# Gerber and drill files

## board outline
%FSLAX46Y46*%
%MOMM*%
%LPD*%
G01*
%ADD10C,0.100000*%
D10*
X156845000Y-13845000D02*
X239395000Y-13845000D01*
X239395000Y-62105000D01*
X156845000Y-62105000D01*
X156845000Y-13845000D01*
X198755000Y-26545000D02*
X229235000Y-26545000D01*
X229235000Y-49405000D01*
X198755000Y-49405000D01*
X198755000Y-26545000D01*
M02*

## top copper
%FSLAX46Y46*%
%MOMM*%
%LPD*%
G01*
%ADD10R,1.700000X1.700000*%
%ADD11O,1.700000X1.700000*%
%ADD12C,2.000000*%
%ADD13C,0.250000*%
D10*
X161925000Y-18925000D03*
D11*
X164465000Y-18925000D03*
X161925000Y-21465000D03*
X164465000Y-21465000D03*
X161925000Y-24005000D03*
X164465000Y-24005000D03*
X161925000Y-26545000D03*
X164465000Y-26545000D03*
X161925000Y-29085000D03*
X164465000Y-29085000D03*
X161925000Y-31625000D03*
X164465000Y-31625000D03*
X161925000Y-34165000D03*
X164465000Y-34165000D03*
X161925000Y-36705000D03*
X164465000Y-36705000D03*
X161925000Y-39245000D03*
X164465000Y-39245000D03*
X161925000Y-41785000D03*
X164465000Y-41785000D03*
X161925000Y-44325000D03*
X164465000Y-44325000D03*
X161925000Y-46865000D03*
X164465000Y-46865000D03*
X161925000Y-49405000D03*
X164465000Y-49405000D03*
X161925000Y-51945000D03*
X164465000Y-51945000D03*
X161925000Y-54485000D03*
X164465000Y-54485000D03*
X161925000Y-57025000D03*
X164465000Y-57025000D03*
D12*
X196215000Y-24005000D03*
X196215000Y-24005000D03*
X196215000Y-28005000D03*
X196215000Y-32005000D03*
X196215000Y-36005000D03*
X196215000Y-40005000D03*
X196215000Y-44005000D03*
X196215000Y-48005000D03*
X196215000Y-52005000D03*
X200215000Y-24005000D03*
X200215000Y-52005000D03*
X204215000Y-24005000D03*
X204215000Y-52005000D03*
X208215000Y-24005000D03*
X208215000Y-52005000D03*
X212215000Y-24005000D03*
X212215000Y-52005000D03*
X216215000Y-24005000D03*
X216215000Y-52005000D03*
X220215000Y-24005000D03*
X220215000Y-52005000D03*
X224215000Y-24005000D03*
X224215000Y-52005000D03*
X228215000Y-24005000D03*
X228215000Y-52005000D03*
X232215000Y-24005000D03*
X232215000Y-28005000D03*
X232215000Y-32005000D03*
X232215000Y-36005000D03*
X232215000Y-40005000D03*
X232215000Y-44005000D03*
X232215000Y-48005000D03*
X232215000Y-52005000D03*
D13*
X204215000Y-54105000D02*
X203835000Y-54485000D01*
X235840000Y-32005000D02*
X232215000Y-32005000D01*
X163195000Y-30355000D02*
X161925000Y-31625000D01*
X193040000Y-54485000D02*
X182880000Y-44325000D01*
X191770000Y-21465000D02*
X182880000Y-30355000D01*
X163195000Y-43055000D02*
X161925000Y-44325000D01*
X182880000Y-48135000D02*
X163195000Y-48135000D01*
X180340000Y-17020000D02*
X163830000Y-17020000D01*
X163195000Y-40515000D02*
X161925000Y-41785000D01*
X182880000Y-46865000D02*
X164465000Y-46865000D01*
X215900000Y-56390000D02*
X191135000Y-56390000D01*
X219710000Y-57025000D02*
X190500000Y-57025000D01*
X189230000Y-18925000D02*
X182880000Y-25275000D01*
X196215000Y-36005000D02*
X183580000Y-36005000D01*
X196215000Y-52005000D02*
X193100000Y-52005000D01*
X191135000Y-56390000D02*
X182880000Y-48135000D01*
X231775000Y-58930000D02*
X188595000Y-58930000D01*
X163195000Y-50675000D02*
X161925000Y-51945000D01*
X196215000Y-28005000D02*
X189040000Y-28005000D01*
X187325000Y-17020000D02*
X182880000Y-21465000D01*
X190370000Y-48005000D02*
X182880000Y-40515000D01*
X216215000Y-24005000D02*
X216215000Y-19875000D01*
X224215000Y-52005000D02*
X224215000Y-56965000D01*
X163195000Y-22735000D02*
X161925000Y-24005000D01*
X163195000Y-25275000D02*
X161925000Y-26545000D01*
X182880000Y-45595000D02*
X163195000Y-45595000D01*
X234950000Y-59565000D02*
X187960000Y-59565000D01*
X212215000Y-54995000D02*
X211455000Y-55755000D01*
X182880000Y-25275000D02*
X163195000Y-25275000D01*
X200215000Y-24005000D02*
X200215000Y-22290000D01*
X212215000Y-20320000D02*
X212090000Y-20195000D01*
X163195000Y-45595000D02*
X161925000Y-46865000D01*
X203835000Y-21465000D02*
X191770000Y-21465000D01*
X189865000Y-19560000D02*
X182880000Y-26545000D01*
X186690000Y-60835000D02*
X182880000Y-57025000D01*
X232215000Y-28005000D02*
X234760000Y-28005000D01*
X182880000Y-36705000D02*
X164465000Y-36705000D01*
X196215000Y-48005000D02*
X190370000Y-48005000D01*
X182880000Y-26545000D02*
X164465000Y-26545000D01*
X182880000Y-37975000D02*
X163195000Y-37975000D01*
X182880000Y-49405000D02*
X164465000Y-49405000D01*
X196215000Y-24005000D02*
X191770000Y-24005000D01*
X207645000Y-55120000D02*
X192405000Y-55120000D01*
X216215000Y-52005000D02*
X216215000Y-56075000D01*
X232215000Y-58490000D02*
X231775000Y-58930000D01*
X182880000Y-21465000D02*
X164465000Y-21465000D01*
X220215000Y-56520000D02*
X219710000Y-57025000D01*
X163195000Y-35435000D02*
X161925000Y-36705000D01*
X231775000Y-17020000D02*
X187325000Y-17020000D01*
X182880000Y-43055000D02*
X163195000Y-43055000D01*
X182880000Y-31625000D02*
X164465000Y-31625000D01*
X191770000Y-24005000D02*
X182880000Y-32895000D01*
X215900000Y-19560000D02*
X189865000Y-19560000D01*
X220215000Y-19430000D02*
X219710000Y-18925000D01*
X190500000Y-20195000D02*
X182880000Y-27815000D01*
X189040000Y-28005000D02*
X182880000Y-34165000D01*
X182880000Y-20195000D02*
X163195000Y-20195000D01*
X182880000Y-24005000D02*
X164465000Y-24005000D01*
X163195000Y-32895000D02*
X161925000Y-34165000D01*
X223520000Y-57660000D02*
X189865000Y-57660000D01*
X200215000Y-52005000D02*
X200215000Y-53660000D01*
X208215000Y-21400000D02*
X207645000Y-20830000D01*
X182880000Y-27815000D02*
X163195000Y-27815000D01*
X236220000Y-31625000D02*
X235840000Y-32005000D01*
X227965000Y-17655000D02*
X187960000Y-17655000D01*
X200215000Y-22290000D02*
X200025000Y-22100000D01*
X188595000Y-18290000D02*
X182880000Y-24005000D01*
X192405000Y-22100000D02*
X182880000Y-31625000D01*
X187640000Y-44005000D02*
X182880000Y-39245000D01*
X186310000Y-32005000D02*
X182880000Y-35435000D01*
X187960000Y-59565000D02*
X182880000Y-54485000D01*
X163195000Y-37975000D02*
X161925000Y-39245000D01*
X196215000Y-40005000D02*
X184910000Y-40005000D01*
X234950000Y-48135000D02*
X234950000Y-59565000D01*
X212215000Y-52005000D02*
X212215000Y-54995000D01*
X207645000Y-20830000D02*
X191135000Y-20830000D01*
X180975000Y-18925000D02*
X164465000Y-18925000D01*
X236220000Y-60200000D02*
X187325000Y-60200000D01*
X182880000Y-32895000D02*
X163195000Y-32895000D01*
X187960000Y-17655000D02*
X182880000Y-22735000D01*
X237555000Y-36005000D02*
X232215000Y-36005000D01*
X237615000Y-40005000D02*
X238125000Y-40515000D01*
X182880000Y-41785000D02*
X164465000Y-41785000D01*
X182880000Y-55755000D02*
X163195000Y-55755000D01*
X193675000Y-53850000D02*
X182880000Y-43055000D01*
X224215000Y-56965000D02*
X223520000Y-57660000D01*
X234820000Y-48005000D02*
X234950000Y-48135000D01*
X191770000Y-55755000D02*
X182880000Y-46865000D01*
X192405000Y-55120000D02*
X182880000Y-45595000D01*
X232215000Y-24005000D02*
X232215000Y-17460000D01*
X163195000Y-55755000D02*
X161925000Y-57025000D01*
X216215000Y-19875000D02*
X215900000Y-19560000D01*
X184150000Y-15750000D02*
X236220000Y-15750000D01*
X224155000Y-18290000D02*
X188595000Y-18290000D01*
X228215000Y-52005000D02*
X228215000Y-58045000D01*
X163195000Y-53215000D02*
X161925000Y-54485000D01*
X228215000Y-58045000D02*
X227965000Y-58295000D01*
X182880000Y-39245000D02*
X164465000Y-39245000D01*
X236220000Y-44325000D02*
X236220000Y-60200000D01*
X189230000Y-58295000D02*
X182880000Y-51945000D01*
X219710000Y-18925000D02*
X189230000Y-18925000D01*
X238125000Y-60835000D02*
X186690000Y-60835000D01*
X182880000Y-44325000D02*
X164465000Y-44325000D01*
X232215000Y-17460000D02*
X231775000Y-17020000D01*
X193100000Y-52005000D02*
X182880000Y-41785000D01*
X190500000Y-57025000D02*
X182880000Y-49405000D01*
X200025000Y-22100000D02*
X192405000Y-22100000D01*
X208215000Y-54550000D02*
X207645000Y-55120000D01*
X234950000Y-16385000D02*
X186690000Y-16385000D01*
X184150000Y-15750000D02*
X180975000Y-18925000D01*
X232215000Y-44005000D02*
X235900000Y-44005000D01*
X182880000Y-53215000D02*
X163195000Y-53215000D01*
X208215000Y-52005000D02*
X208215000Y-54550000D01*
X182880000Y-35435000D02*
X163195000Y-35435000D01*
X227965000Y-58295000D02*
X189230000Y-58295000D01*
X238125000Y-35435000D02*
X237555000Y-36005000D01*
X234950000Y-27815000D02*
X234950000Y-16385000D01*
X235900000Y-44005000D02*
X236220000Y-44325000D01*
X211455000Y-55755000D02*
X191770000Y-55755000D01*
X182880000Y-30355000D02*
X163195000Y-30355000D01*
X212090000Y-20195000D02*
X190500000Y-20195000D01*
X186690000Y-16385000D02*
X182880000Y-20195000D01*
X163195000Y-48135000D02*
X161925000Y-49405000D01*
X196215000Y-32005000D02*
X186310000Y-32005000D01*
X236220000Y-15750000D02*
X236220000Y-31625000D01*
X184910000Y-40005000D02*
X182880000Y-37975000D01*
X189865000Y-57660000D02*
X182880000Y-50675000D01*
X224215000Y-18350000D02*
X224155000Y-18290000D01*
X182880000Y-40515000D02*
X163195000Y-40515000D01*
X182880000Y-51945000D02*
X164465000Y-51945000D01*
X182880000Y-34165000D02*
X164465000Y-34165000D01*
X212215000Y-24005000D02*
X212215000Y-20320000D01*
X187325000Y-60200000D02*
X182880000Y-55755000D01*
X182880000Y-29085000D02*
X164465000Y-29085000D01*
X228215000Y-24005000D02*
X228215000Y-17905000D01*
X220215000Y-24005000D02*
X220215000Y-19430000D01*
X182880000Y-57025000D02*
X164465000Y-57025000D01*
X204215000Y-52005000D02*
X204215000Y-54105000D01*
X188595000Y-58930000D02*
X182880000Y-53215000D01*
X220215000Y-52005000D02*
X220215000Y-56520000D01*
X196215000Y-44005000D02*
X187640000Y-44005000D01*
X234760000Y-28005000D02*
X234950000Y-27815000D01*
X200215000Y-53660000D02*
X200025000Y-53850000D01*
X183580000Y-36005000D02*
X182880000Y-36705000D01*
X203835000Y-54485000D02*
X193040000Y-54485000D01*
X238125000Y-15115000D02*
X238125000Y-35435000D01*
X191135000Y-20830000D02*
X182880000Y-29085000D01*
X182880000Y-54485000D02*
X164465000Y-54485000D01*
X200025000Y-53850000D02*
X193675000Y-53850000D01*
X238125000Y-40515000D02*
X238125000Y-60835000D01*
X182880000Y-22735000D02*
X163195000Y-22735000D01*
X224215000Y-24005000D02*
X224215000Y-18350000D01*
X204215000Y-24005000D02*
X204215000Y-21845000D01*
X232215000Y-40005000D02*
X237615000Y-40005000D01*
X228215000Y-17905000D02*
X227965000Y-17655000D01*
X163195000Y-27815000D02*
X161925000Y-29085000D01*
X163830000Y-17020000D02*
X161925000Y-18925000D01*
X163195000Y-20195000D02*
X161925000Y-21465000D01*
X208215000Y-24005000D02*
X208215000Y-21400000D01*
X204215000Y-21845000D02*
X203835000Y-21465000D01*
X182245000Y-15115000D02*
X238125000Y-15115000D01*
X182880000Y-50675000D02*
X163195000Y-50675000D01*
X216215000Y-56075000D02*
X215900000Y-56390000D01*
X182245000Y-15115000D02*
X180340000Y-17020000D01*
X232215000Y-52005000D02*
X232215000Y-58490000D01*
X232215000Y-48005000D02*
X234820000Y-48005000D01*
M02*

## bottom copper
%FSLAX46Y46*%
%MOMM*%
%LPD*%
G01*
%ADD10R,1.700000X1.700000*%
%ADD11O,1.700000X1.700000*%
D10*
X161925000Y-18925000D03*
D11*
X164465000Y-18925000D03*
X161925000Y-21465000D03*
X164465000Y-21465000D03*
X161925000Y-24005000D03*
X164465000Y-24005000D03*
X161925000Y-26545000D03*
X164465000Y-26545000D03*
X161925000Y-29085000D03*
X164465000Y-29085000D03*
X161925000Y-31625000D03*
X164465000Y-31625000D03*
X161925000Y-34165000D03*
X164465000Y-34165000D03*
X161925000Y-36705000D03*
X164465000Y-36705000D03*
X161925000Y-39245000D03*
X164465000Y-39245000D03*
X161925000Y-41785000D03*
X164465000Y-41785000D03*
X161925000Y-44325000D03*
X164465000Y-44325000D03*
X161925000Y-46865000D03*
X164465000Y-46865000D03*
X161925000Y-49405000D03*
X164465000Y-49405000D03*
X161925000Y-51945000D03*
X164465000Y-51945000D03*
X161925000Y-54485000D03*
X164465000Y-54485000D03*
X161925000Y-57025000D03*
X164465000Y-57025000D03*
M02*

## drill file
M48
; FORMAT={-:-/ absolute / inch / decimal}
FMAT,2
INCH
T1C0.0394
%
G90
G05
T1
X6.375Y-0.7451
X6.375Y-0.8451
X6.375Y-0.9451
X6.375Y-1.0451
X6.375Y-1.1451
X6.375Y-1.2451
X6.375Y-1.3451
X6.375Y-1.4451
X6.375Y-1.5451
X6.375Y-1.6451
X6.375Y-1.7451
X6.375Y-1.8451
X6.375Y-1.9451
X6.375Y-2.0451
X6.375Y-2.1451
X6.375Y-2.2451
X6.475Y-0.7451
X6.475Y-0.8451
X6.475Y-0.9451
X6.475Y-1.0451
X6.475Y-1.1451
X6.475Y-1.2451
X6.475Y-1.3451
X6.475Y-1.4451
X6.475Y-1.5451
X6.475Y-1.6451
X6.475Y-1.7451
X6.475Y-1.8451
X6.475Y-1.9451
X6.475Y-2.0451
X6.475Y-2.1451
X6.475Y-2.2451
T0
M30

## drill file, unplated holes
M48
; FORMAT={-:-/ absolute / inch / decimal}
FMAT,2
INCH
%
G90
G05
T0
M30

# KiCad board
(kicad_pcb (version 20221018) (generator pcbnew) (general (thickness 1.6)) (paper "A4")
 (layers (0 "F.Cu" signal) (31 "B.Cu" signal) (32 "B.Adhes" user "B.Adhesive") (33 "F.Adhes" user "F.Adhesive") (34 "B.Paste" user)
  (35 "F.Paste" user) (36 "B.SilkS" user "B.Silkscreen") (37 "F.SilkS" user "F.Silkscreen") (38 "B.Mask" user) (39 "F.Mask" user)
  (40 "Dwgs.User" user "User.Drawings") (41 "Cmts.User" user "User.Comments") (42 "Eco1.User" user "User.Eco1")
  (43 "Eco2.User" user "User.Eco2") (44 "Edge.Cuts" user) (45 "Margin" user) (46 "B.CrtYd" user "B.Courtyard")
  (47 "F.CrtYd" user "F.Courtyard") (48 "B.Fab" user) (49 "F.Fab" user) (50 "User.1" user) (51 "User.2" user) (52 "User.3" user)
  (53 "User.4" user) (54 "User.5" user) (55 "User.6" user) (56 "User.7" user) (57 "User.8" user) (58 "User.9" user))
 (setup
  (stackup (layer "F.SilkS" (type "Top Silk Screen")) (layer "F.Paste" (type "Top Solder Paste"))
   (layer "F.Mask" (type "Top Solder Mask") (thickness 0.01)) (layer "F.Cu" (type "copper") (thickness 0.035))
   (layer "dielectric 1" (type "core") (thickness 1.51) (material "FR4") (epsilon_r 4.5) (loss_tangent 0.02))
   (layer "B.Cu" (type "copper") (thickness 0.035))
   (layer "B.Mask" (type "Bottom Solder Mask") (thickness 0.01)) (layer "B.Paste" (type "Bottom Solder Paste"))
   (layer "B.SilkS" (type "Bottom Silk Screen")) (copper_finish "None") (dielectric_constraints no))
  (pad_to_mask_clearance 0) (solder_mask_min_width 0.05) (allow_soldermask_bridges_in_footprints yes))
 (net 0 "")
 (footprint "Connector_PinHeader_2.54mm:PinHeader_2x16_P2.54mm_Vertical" (layer "F.Cu") (at 161.925 18.925)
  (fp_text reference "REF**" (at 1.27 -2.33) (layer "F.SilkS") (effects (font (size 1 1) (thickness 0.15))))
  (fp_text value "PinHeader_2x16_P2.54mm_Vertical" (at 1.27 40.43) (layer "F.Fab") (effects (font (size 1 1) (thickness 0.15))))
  (pad "1" thru_hole rect (at 0 0) (size 1.7 1.7) (drill 1) (layers "*.Cu" "*.Mask"))
  (pad "2" thru_hole oval (at 2.54 0) (size 1.7 1.7) (drill 1) (layers "*.Cu" "*.Mask"))
  (pad "3" thru_hole oval (at 0 2.54) (size 1.7 1.7) (drill 1) (layers "*.Cu" "*.Mask"))
  (pad "4" thru_hole oval (at 2.54 2.54) (size 1.7 1.7) (drill 1) (layers "*.Cu" "*.Mask"))
  (pad "5" thru_hole oval (at 0 5.08) (size 1.7 1.7) (drill 1) (layers "*.Cu" "*.Mask"))
  (pad "6" thru_hole oval (at 2.54 5.08) (size 1.7 1.7) (drill 1) (layers "*.Cu" "*.Mask"))
  (pad "7" thru_hole oval (at 0 7.62) (size 1.7 1.7) (drill 1) (layers "*.Cu" "*.Mask"))
  (pad "8" thru_hole oval (at 2.54 7.62) (size 1.7 1.7) (drill 1) (layers "*.Cu" "*.Mask"))
  (pad "9" thru_hole oval (at 0 10.16) (size 1.7 1.7) (drill 1) (layers "*.Cu" "*.Mask"))
  (pad "10" thru_hole oval (at 2.54 10.16) (size 1.7 1.7) (drill 1) (layers "*.Cu" "*.Mask"))
  (pad "11" thru_hole oval (at 0 12.7) (size 1.7 1.7) (drill 1) (layers "*.Cu" "*.Mask") (clearance 0.2))
  (pad "12" thru_hole oval (at 2.54 12.7) (size 1.7 1.7) (drill 1) (layers "*.Cu" "*.Mask"))
  (pad "13" thru_hole oval (at 0 15.24) (size 1.7 1.7) (drill 1) (layers "*.Cu" "*.Mask"))
  (pad "14" thru_hole oval (at 2.54 15.24) (size 1.7 1.7) (drill 1) (layers "*.Cu" "*.Mask"))
  (pad "15" thru_hole oval (at 0 17.78) (size 1.7 1.7) (drill 1) (layers "*.Cu" "*.Mask"))
  (pad "16" thru_hole oval (at 2.54 17.78) (size 1.7 1.7) (drill 1) (layers "*.Cu" "*.Mask"))
  (pad "17" thru_hole oval (at 0 20.32) (size 1.7 1.7) (drill 1) (layers "*.Cu" "*.Mask"))
  (pad "18" thru_hole oval (at 2.54 20.32) (size 1.7 1.7) (drill 1) (layers "*.Cu" "*.Mask"))
  (pad "19" thru_hole oval (at 0 22.86) (size 1.7 1.7) (drill 1) (layers "*.Cu" "*.Mask"))
  (pad "20" thru_hole oval (at 2.54 22.86) (size 1.7 1.7) (drill 1) (layers "*.Cu" "*.Mask"))
  (pad "21" thru_hole oval (at 0 25.4) (size 1.7 1.7) (drill 1) (layers "*.Cu" "*.Mask"))
  (pad "22" thru_hole oval (at 2.54 25.4) (size 1.7 1.7) (drill 1) (layers "*.Cu" "*.Mask"))
  (pad "23" thru_hole oval (at 0 27.94) (size 1.7 1.7) (drill 1) (layers "*.Cu" "*.Mask"))
  (pad "24" thru_hole oval (at 2.54 27.94) (size 1.7 1.7) (drill 1) (layers "*.Cu" "*.Mask"))
  (pad "25" thru_hole oval (at 0 30.48) (size 1.7 1.7) (drill 1) (layers "*.Cu" "*.Mask"))
  (pad "26" thru_hole oval (at 2.54 30.48) (size 1.7 1.7) (drill 1) (layers "*.Cu" "*.Mask"))
  (pad "27" thru_hole oval (at 0 33.02) (size 1.7 1.7) (drill 1) (layers "*.Cu" "*.Mask"))
  (pad "28" thru_hole oval (at 2.54 33.02) (size 1.7 1.7) (drill 1) (layers "*.Cu" "*.Mask"))
  (pad "29" thru_hole oval (at 0 35.56) (size 1.7 1.7) (drill 1) (layers "*.Cu" "*.Mask"))
  (pad "30" thru_hole oval (at 2.54 35.56) (size 1.7 1.7) (drill 1) (layers "*.Cu" "*.Mask"))
  (pad "31" thru_hole oval (at 0 38.1) (size 1.7 1.7) (drill 1) (layers "*.Cu" "*.Mask"))
  (pad "32" thru_hole oval (at 2.54 38.1) (size 1.7 1.7) (drill 1) (layers "*.Cu" "*.Mask")))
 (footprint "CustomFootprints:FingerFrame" (layer "F.Cu") (at 196.215 24.005)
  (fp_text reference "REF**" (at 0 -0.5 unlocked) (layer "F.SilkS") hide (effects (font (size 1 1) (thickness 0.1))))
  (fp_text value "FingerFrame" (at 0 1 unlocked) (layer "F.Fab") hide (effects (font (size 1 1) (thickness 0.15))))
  (pad "1" smd circle (at 0 0) (size 2 2) (layers "F.Cu" "F.Paste" "F.Mask"))
  (pad "1" smd circle (at 0 0) (size 2 2) (layers "F.Cu" "F.Paste" "F.Mask"))
  (pad "1" smd circle (at 0 4) (size 2 2) (layers "F.Cu" "F.Paste" "F.Mask"))
  (pad "1" smd circle (at 0 8) (size 2 2) (layers "F.Cu" "F.Paste" "F.Mask"))
  (pad "1" smd circle (at 0 12) (size 2 2) (layers "F.Cu" "F.Paste" "F.Mask"))
  (pad "1" smd circle (at 0 16) (size 2 2) (layers "F.Cu" "F.Paste" "F.Mask"))
  (pad "1" smd circle (at 0 20) (size 2 2) (layers "F.Cu" "F.Paste" "F.Mask"))
  (pad "1" smd circle (at 0 24) (size 2 2) (layers "F.Cu" "F.Paste" "F.Mask"))
  (pad "1" smd circle (at 0 28) (size 2 2) (layers "F.Cu" "F.Paste" "F.Mask"))
  (pad "1" smd circle (at 4 0) (size 2 2) (layers "F.Cu" "F.Paste" "F.Mask"))
  (pad "1" smd circle (at 4 28) (size 2 2) (layers "F.Cu" "F.Paste" "F.Mask"))
  (pad "1" smd circle (at 8 0) (size 2 2) (layers "F.Cu" "F.Paste" "F.Mask"))
  (pad "1" smd circle (at 8 28) (size 2 2) (layers "F.Cu" "F.Paste" "F.Mask"))
  (pad "1" smd circle (at 12 0) (size 2 2) (layers "F.Cu" "F.Paste" "F.Mask"))
  (pad "1" smd circle (at 12 28) (size 2 2) (layers "F.Cu" "F.Paste" "F.Mask"))
  (pad "1" smd circle (at 16 0) (size 2 2) (layers "F.Cu" "F.Paste" "F.Mask"))
  (pad "1" smd circle (at 16 28) (size 2 2) (layers "F.Cu" "F.Paste" "F.Mask"))
  (pad "1" smd circle (at 20 0) (size 2 2) (layers "F.Cu" "F.Paste" "F.Mask"))
  (pad "1" smd circle (at 20 28) (size 2 2) (layers "F.Cu" "F.Paste" "F.Mask"))
  (pad "1" smd circle (at 24 0) (size 2 2) (layers "F.Cu" "F.Paste" "F.Mask"))
  (pad "1" smd circle (at 24 28) (size 2 2) (layers "F.Cu" "F.Paste" "F.Mask"))
  (pad "1" smd circle (at 28 0) (size 2 2) (layers "F.Cu" "F.Paste" "F.Mask"))
  (pad "1" smd circle (at 28 28) (size 2 2) (layers "F.Cu" "F.Paste" "F.Mask"))
  (pad "1" smd circle (at 32 0) (size 2 2) (layers "F.Cu" "F.Paste" "F.Mask"))
  (pad "1" smd circle (at 32 28) (size 2 2) (layers "F.Cu" "F.Paste" "F.Mask"))
  (pad "1" smd circle (at 36 0) (size 2 2) (layers "F.Cu" "F.Paste" "F.Mask"))
  (pad "1" smd circle (at 36 4) (size 2 2) (layers "F.Cu" "F.Paste" "F.Mask"))
  (pad "1" smd circle (at 36 8) (size 2 2) (layers "F.Cu" "F.Paste" "F.Mask"))
  (pad "1" smd circle (at 36 12) (size 2 2) (layers "F.Cu" "F.Paste" "F.Mask"))
  (pad "1" smd circle (at 36 16) (size 2 2) (layers "F.Cu" "F.Paste" "F.Mask"))
  (pad "1" smd circle (at 36 20) (size 2 2) (layers "F.Cu" "F.Paste" "F.Mask"))
  (pad "1" smd circle (at 36 24) (size 2 2) (layers "F.Cu" "F.Paste" "F.Mask"))
  (pad "1" smd circle (at 36 28) (size 2 2) (layers "F.Cu" "F.Paste" "F.Mask")))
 (gr_rect (start 156.845 13.845) (end 239.395 62.105) (stroke (width 0.1) (type default)) (fill none) (layer "Edge.Cuts"))
 (gr_rect (start 198.755 26.545) (end 229.235 49.405) (stroke (width 0.1) (type default)) (fill none) (layer "Edge.Cuts"))
 (segment (start 204.215 54.105) (end 203.835 54.485) (width 0.25) (layer "F.Cu") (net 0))
 (segment (start 235.84 32.005) (end 232.215 32.005) (width 0.25) (layer "F.Cu") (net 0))
 (segment (start 163.195 30.355) (end 161.925 31.625) (width 0.25) (layer "F.Cu") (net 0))
 (segment (start 193.04 54.485) (end 182.88 44.325) (width 0.25) (layer "F.Cu") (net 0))
 (segment (start 191.77 21.465) (end 182.88 30.355) (width 0.25) (layer "F.Cu") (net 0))
 (segment (start 163.195 43.055) (end 161.925 44.325) (width 0.25) (layer "F.Cu") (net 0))
 (segment (start 182.88 48.135) (end 163.195 48.135) (width 0.25) (layer "F.Cu") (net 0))
 (segment (start 180.34 17.02) (end 163.83 17.02) (width 0.25) (layer "F.Cu") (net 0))
 (segment (start 163.195 40.515) (end 161.925 41.785) (width 0.25) (layer "F.Cu") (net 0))
 (segment (start 182.88 46.865) (end 164.465 46.865) (width 0.25) (layer "F.Cu") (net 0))
 (segment (start 215.9 56.39) (end 191.135 56.39) (width 0.25) (layer "F.Cu") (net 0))
 (segment (start 219.71 57.025) (end 190.5 57.025) (width 0.25) (layer "F.Cu") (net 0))
 (segment (start 189.23 18.925) (end 182.88 25.275) (width 0.25) (layer "F.Cu") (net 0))
 (segment (start 196.215 36.005) (end 183.58 36.005) (width 0.25) (layer "F.Cu") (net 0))
 (segment (start 196.215 52.005) (end 193.1 52.005) (width 0.25) (layer "F.Cu") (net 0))
 (segment (start 191.135 56.39) (end 182.88 48.135) (width 0.25) (layer "F.Cu") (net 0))
 (segment (start 231.775 58.93) (end 188.595 58.93) (width 0.25) (layer "F.Cu") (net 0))
 (segment (start 163.195 50.675) (end 161.925 51.945) (width 0.25) (layer "F.Cu") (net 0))
 (segment (start 196.215 28.005) (end 189.04 28.005) (width 0.25) (layer "F.Cu") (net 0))
 (segment (start 187.325 17.02) (end 182.88 21.465) (width 0.25) (layer "F.Cu") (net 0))
 (segment (start 190.37 48.005) (end 182.88 40.515) (width 0.25) (layer "F.Cu") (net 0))
 (segment (start 216.215 24.005) (end 216.215 19.875) (width 0.25) (layer "F.Cu") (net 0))
 (segment (start 224.215 52.005) (end 224.215 56.965) (width 0.25) (layer "F.Cu") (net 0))
 (segment (start 163.195 22.735) (end 161.925 24.005) (width 0.25) (layer "F.Cu") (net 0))
 (segment (start 163.195 25.275) (end 161.925 26.545) (width 0.25) (layer "F.Cu") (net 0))
 (segment (start 182.88 45.595) (end 163.195 45.595) (width 0.25) (layer "F.Cu") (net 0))
 (segment (start 234.95 59.565) (end 187.96 59.565) (width 0.25) (layer "F.Cu") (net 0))
 (segment (start 212.215 54.995) (end 211.455 55.755) (width 0.25) (layer "F.Cu") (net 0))
 (segment (start 182.88 25.275) (end 163.195 25.275) (width 0.25) (layer "F.Cu") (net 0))
 (segment (start 200.215 24.005) (end 200.215 22.29) (width 0.25) (layer "F.Cu") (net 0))
 (segment (start 212.215 20.32) (end 212.09 20.195) (width 0.25) (layer "F.Cu") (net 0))
 (segment (start 163.195 45.595) (end 161.925 46.865) (width 0.25) (layer "F.Cu") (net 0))
 (segment (start 203.835 21.465) (end 191.77 21.465) (width 0.25) (layer "F.Cu") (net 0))
 (segment (start 189.865 19.56) (end 182.88 26.545) (width 0.25) (layer "F.Cu") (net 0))
 (segment (start 186.69 60.835) (end 182.88 57.025) (width 0.25) (layer "F.Cu") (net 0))
 (segment (start 232.215 28.005) (end 234.76 28.005) (width 0.25) (layer "F.Cu") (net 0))
 (segment (start 182.88 36.705) (end 164.465 36.705) (width 0.25) (layer "F.Cu") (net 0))
 (segment (start 196.215 48.005) (end 190.37 48.005) (width 0.25) (layer "F.Cu") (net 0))
 (segment (start 182.88 26.545) (end 164.465 26.545) (width 0.25) (layer "F.Cu") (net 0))
 (segment (start 182.88 37.975) (end 163.195 37.975) (width 0.25) (layer "F.Cu") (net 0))
 (segment (start 182.88 49.405) (end 164.465 49.405) (width 0.25) (layer "F.Cu") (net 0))
 (segment (start 196.215 24.005) (end 191.77 24.005) (width 0.25) (layer "F.Cu") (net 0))
 (segment (start 207.645 55.12) (end 192.405 55.12) (width 0.25) (layer "F.Cu") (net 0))
 (segment (start 216.215 52.005) (end 216.215 56.075) (width 0.25) (layer "F.Cu") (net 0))
 (segment (start 232.215 58.49) (end 231.775 58.93) (width 0.25) (layer "F.Cu") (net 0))
 (segment (start 182.88 21.465) (end 164.465 21.465) (width 0.25) (layer "F.Cu") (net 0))
 (segment (start 220.215 56.52) (end 219.71 57.025) (width 0.25) (layer "F.Cu") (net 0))
 (segment (start 163.195 35.435) (end 161.925 36.705) (width 0.25) (layer "F.Cu") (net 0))
 (segment (start 231.775 17.02) (end 187.325 17.02) (width 0.25) (layer "F.Cu") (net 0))
 (segment (start 182.88 43.055) (end 163.195 43.055) (width 0.25) (layer "F.Cu") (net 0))
 (segment (start 182.88 31.625) (end 164.465 31.625) (width 0.25) (layer "F.Cu") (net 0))
 (segment (start 191.77 24.005) (end 182.88 32.895) (width 0.25) (layer "F.Cu") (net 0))
 (segment (start 215.9 19.56) (end 189.865 19.56) (width 0.25) (layer "F.Cu") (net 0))
 (segment (start 220.215 19.43) (end 219.71 18.925) (width 0.25) (layer "F.Cu") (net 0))
 (segment (start 190.5 20.195) (end 182.88 27.815) (width 0.25) (layer "F.Cu") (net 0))
 (segment (start 189.04 28.005) (end 182.88 34.165) (width 0.25) (layer "F.Cu") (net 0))
 (segment (start 182.88 20.195) (end 163.195 20.195) (width 0.25) (layer "F.Cu") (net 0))
 (segment (start 182.88 24.005) (end 164.465 24.005) (width 0.25) (layer "F.Cu") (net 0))
 (segment (start 163.195 32.895) (end 161.925 34.165) (width 0.25) (layer "F.Cu") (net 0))
 (segment (start 223.52 57.66) (end 189.865 57.66) (width 0.25) (layer "F.Cu") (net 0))
 (segment (start 200.215 52.005) (end 200.215 53.66) (width 0.25) (layer "F.Cu") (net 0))
 (segment (start 208.215 21.4) (end 207.645 20.83) (width 0.25) (layer "F.Cu") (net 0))
 (segment (start 182.88 27.815) (end 163.195 27.815) (width 0.25) (layer "F.Cu") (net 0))
 (segment (start 236.22 31.625) (end 235.84 32.005) (width 0.25) (layer "F.Cu") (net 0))
 (segment (start 227.965 17.655) (end 187.96 17.655) (width 0.25) (layer "F.Cu") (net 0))
 (segment (start 200.215 22.29) (end 200.025 22.1) (width 0.25) (layer "F.Cu") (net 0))
 (segment (start 188.595 18.29) (end 182.88 24.005) (width 0.25) (layer "F.Cu") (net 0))
 (segment (start 192.405 22.1) (end 182.88 31.625) (width 0.25) (layer "F.Cu") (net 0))
 (segment (start 187.64 44.005) (end 182.88 39.245) (width 0.25) (layer "F.Cu") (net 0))
 (segment (start 186.31 32.005) (end 182.88 35.435) (width 0.25) (layer "F.Cu") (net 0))
 (segment (start 187.96 59.565) (end 182.88 54.485) (width 0.25) (layer "F.Cu") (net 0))
 (segment (start 163.195 37.975) (end 161.925 39.245) (width 0.25) (layer "F.Cu") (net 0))
 (segment (start 196.215 40.005) (end 184.91 40.005) (width 0.25) (layer "F.Cu") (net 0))
 (segment (start 234.95 48.135) (end 234.95 59.565) (width 0.25) (layer "F.Cu") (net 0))
 (segment (start 212.215 52.005) (end 212.215 54.995) (width 0.25) (layer "F.Cu") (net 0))
 (segment (start 207.645 20.83) (end 191.135 20.83) (width 0.25) (layer "F.Cu") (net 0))
 (segment (start 180.975 18.925) (end 164.465 18.925) (width 0.25) (layer "F.Cu") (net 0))
 (segment (start 236.22 60.2) (end 187.325 60.2) (width 0.25) (layer "F.Cu") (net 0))
 (segment (start 182.88 32.895) (end 163.195 32.895) (width 0.25) (layer "F.Cu") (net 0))
 (segment (start 187.96 17.655) (end 182.88 22.735) (width 0.25) (layer "F.Cu") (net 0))
 (segment (start 237.555 36.005) (end 232.215 36.005) (width 0.25) (layer "F.Cu") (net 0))
 (segment (start 237.615 40.005) (end 238.125 40.515) (width 0.25) (layer "F.Cu") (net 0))
 (segment (start 182.88 41.785) (end 164.465 41.785) (width 0.25) (layer "F.Cu") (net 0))
 (segment (start 182.88 55.755) (end 163.195 55.755) (width 0.25) (layer "F.Cu") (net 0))
 (segment (start 193.675 53.85) (end 182.88 43.055) (width 0.25) (layer "F.Cu") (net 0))
 (segment (start 224.215 56.965) (end 223.52 57.66) (width 0.25) (layer "F.Cu") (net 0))
 (segment (start 234.82 48.005) (end 234.95 48.135) (width 0.25) (layer "F.Cu") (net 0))
 (segment (start 191.77 55.755) (end 182.88 46.865) (width 0.25) (layer "F.Cu") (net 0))
 (segment (start 192.405 55.12) (end 182.88 45.595) (width 0.25) (layer "F.Cu") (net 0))
 (segment (start 232.215 24.005) (end 232.215 17.46) (width 0.25) (layer "F.Cu") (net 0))
 (segment (start 163.195 55.755) (end 161.925 57.025) (width 0.25) (layer "F.Cu") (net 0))
 (segment (start 216.215 19.875) (end 215.9 19.56) (width 0.25) (layer "F.Cu") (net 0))
 (segment (start 184.15 15.75) (end 236.22 15.75) (width 0.25) (layer "F.Cu") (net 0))
 (segment (start 224.155 18.29) (end 188.595 18.29) (width 0.25) (layer "F.Cu") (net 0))
 (segment (start 228.215 52.005) (end 228.215 58.045) (width 0.25) (layer "F.Cu") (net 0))
 (segment (start 163.195 53.215) (end 161.925 54.485) (width 0.25) (layer "F.Cu") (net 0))
 (segment (start 228.215 58.045) (end 227.965 58.295) (width 0.25) (layer "F.Cu") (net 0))
 (segment (start 182.88 39.245) (end 164.465 39.245) (width 0.25) (layer "F.Cu") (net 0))
 (segment (start 236.22 44.325) (end 236.22 60.2) (width 0.25) (layer "F.Cu") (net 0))
 (segment (start 189.23 58.295) (end 182.88 51.945) (width 0.25) (layer "F.Cu") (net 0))
 (segment (start 219.71 18.925) (end 189.23 18.925) (width 0.25) (layer "F.Cu") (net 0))
 (segment (start 238.125 60.835) (end 186.69 60.835) (width 0.25) (layer "F.Cu") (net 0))
 (segment (start 182.88 44.325) (end 164.465 44.325) (width 0.25) (layer "F.Cu") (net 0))
 (segment (start 232.215 17.46) (end 231.775 17.02) (width 0.25) (layer "F.Cu") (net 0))
 (segment (start 193.1 52.005) (end 182.88 41.785) (width 0.25) (layer "F.Cu") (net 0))
 (segment (start 190.5 57.025) (end 182.88 49.405) (width 0.25) (layer "F.Cu") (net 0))
 (segment (start 200.025 22.1) (end 192.405 22.1) (width 0.25) (layer "F.Cu") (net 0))
 (segment (start 208.215 54.55) (end 207.645 55.12) (width 0.25) (layer "F.Cu") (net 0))
 (segment (start 234.95 16.385) (end 186.69 16.385) (width 0.25) (layer "F.Cu") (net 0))
 (segment (start 184.15 15.75) (end 180.975 18.925) (width 0.25) (layer "F.Cu") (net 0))
 (segment (start 232.215 44.005) (end 235.9 44.005) (width 0.25) (layer "F.Cu") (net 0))
 (segment (start 182.88 53.215) (end 163.195 53.215) (width 0.25) (layer "F.Cu") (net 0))
 (segment (start 208.215 52.005) (end 208.215 54.55) (width 0.25) (layer "F.Cu") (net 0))
 (segment (start 182.88 35.435) (end 163.195 35.435) (width 0.25) (layer "F.Cu") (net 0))
 (segment (start 227.965 58.295) (end 189.23 58.295) (width 0.25) (layer "F.Cu") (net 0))
 (segment (start 238.125 35.435) (end 237.555 36.005) (width 0.25) (layer "F.Cu") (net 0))
 (segment (start 234.95 27.815) (end 234.95 16.385) (width 0.25) (layer "F.Cu") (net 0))
 (segment (start 235.9 44.005) (end 236.22 44.325) (width 0.25) (layer "F.Cu") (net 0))
 (segment (start 211.455 55.755) (end 191.77 55.755) (width 0.25) (layer "F.Cu") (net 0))
 (segment (start 182.88 30.355) (end 163.195 30.355) (width 0.25) (layer "F.Cu") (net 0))
 (segment (start 212.09 20.195) (end 190.5 20.195) (width 0.25) (layer "F.Cu") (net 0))
 (segment (start 186.69 16.385) (end 182.88 20.195) (width 0.25) (layer "F.Cu") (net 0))
 (segment (start 163.195 48.135) (end 161.925 49.405) (width 0.25) (layer "F.Cu") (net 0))
 (segment (start 196.215 32.005) (end 186.31 32.005) (width 0.25) (layer "F.Cu") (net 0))
 (segment (start 236.22 15.75) (end 236.22 31.625) (width 0.25) (layer "F.Cu") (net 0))
 (segment (start 184.91 40.005) (end 182.88 37.975) (width 0.25) (layer "F.Cu") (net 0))
 (segment (start 189.865 57.66) (end 182.88 50.675) (width 0.25) (layer "F.Cu") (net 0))
 (segment (start 224.215 18.35) (end 224.155 18.29) (width 0.25) (layer "F.Cu") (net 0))
 (segment (start 182.88 40.515) (end 163.195 40.515) (width 0.25) (layer "F.Cu") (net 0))
 (segment (start 182.88 51.945) (end 164.465 51.945) (width 0.25) (layer "F.Cu") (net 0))
 (segment (start 182.88 34.165) (end 164.465 34.165) (width 0.25) (layer "F.Cu") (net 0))
 (segment (start 212.215 24.005) (end 212.215 20.32) (width 0.25) (layer "F.Cu") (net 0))
 (segment (start 187.325 60.2) (end 182.88 55.755) (width 0.25) (layer "F.Cu") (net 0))
 (segment (start 182.88 29.085) (end 164.465 29.085) (width 0.25) (layer "F.Cu") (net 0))
 (segment (start 228.215 24.005) (end 228.215 17.905) (width 0.25) (layer "F.Cu") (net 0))
 (segment (start 220.215 24.005) (end 220.215 19.43) (width 0.25) (layer "F.Cu") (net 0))
 (segment (start 182.88 57.025) (end 164.465 57.025) (width 0.25) (layer "F.Cu") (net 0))
 (segment (start 204.215 52.005) (end 204.215 54.105) (width 0.25) (layer "F.Cu") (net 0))
 (segment (start 188.595 58.93) (end 182.88 53.215) (width 0.25) (layer "F.Cu") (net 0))
 (segment (start 220.215 52.005) (end 220.215 56.52) (width 0.25) (layer "F.Cu") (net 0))
 (segment (start 196.215 44.005) (end 187.64 44.005) (width 0.25) (layer "F.Cu") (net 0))
 (segment (start 234.76 28.005) (end 234.95 27.815) (width 0.25) (layer "F.Cu") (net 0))
 (segment (start 200.215 53.66) (end 200.025 53.85) (width 0.25) (layer "F.Cu") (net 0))
 (segment (start 183.58 36.005) (end 182.88 36.705) (width 0.25) (layer "F.Cu") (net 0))
 (segment (start 203.835 54.485) (end 193.04 54.485) (width 0.25) (layer "F.Cu") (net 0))
 (segment (start 238.125 15.115) (end 238.125 35.435) (width 0.25) (layer "F.Cu") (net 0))
 (segment (start 191.135 20.83) (end 182.88 29.085) (width 0.25) (layer "F.Cu") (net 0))
 (segment (start 182.88 54.485) (end 164.465 54.485) (width 0.25) (layer "F.Cu") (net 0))
 (segment (start 200.025 53.85) (end 193.675 53.85) (width 0.25) (layer "F.Cu") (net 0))
 (segment (start 238.125 40.515) (end 238.125 60.835) (width 0.25) (layer "F.Cu") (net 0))
 (segment (start 182.88 22.735) (end 163.195 22.735) (width 0.25) (layer "F.Cu") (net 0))
 (segment (start 224.215 24.005) (end 224.215 18.35) (width 0.25) (layer "F.Cu") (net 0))
 (segment (start 204.215 24.005) (end 204.215 21.845) (width 0.25) (layer "F.Cu") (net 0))
 (segment (start 232.215 40.005) (end 237.615 40.005) (width 0.25) (layer "F.Cu") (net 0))
 (segment (start 228.215 17.905) (end 227.965 17.655) (width 0.25) (layer "F.Cu") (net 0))
 (segment (start 163.195 27.815) (end 161.925 29.085) (width 0.25) (layer "F.Cu") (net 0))
 (segment (start 163.83 17.02) (end 161.925 18.925) (width 0.25) (layer "F.Cu") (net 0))
 (segment (start 163.195 20.195) (end 161.925 21.465) (width 0.25) (layer "F.Cu") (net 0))
 (segment (start 208.215 24.005) (end 208.215 21.4) (width 0.25) (layer "F.Cu") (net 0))
 (segment (start 204.215 21.845) (end 203.835 21.465) (width 0.25) (layer "F.Cu") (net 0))
 (segment (start 182.245 15.115) (end 238.125 15.115) (width 0.25) (layer "F.Cu") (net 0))
 (segment (start 182.88 50.675) (end 163.195 50.675) (width 0.25) (layer "F.Cu") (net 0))
 (segment (start 216.215 56.075) (end 215.9 56.39) (width 0.25) (layer "F.Cu") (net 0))
 (segment (start 182.245 15.115) (end 180.34 17.02) (width 0.25) (layer "F.Cu") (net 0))
 (segment (start 232.215 52.005) (end 232.215 58.49) (width 0.25) (layer "F.Cu") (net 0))
 (segment (start 232.215 48.005) (end 234.82 48.005) (width 0.25) (layer "F.Cu") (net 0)))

